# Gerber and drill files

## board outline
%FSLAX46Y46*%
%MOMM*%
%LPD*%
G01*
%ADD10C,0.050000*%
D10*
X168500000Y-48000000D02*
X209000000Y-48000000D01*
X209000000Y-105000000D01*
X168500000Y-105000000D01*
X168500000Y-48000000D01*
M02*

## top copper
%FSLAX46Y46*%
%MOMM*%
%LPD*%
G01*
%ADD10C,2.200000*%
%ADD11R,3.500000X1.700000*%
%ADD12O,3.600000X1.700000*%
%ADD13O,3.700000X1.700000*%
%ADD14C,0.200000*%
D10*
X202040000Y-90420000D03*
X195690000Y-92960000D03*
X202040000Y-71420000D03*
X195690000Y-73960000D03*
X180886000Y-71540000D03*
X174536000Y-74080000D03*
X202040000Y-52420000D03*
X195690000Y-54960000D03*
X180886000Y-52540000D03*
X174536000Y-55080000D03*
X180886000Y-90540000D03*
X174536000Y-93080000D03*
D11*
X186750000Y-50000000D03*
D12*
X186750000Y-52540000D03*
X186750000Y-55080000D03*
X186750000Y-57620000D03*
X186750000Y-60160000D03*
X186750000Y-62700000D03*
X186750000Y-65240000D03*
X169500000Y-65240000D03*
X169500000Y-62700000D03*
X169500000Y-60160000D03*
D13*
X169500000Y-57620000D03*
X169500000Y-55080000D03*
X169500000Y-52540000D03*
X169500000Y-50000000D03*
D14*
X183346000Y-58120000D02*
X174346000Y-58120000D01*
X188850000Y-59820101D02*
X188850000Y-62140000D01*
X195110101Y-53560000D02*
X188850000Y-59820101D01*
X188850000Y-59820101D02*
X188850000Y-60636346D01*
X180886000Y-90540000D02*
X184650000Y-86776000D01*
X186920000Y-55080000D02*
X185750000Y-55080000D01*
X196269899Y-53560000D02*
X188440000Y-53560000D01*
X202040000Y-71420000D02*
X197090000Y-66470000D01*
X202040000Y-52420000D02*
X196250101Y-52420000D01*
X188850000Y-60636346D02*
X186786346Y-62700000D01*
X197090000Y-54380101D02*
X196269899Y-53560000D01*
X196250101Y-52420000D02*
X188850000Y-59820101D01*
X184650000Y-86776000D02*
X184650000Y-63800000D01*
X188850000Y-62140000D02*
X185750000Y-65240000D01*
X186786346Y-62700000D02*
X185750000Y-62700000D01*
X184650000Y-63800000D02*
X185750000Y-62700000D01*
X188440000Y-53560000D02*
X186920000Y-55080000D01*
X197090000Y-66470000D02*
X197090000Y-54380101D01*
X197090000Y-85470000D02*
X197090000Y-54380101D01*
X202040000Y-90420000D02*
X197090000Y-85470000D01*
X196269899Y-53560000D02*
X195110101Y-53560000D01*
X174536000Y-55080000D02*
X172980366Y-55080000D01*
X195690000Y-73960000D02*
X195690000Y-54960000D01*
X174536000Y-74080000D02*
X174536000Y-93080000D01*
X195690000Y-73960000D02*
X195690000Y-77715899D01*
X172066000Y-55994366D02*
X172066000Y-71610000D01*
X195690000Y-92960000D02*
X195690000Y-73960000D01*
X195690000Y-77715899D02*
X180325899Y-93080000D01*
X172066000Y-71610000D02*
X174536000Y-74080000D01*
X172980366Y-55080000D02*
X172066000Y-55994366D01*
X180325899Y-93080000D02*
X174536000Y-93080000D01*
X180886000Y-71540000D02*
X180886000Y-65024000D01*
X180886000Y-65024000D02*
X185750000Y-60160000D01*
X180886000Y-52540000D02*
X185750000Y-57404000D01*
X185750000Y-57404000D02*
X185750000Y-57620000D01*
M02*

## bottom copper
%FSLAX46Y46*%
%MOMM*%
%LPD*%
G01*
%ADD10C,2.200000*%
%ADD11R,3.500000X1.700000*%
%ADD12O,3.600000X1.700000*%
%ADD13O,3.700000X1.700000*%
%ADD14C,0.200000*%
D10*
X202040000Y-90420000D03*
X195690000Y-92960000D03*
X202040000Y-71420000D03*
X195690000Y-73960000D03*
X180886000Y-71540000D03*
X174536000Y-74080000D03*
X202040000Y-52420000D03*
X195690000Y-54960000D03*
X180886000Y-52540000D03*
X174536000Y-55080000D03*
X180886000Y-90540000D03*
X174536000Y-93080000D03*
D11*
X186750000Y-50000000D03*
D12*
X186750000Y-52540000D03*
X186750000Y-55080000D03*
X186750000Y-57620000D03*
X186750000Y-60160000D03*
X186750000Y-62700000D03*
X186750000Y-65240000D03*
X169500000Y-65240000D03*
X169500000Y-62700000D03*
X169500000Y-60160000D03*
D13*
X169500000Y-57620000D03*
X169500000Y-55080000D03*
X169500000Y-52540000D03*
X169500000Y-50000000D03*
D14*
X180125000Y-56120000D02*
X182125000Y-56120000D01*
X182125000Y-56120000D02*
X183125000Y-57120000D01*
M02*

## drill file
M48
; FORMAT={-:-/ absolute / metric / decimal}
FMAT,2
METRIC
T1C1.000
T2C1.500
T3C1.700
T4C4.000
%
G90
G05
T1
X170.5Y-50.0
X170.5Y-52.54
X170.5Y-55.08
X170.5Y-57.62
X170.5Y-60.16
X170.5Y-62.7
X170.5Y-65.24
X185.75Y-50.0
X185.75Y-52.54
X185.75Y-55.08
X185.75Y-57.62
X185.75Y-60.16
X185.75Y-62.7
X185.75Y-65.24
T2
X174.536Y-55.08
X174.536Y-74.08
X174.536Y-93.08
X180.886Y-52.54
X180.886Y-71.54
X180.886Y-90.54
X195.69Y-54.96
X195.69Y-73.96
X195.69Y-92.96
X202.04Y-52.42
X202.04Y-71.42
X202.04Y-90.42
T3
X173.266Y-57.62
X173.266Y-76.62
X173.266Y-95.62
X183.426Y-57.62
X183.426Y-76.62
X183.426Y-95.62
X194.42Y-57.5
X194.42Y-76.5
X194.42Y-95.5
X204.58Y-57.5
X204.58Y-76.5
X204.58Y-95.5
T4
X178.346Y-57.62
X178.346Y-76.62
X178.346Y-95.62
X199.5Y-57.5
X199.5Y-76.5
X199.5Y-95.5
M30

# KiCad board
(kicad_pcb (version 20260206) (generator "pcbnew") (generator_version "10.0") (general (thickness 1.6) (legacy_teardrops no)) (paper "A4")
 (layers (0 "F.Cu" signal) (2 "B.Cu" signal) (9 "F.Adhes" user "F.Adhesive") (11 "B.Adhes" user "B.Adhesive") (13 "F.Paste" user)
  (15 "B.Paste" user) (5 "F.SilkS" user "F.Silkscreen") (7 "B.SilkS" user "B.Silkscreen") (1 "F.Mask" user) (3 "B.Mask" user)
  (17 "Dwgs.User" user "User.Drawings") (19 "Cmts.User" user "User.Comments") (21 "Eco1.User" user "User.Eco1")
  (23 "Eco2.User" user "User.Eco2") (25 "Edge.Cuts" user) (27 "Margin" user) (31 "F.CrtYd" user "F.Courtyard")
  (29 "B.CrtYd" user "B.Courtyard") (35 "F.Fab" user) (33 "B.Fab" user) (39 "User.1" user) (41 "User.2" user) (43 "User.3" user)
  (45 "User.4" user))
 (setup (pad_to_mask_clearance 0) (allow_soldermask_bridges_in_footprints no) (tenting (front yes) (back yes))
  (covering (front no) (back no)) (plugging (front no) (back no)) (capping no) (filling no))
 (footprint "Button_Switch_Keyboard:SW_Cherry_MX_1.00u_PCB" (layer "F.Cu") (at 202.04 90.42)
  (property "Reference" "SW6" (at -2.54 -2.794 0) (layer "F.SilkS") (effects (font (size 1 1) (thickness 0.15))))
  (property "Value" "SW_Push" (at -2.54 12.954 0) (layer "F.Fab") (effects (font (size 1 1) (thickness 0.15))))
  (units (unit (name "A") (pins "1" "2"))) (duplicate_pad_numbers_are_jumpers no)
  (pad "" np_thru_hole circle (at -7.62 5.08) (size 1.7 1.7) (drill 1.7) (layers "*.Cu" "*.Mask"))
  (pad "" np_thru_hole circle (at -2.54 5.08) (size 4 4) (drill 4) (layers "*.Cu" "*.Mask"))
  (pad "" np_thru_hole circle (at 2.54 5.08) (size 1.7 1.7) (drill 1.7) (layers "*.Cu" "*.Mask"))
  (pad "1" thru_hole circle (at 0 0) (size 2.2 2.2) (drill 1.5) (layers "*.Cu" "*.Mask") (remove_unused_layers no)
   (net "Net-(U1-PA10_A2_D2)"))
  (pad "2" thru_hole circle (at -6.35 2.54) (size 2.2 2.2) (drill 1.5) (layers "*.Cu" "*.Mask") (remove_unused_layers no) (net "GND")))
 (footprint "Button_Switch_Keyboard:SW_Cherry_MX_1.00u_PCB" (layer "F.Cu") (at 202.04 71.42)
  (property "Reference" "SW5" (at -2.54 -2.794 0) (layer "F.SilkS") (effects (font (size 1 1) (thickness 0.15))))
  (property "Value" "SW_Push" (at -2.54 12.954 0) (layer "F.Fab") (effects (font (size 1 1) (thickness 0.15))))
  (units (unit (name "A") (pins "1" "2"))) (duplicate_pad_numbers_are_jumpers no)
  (pad "" np_thru_hole circle (at -7.62 5.08) (size 1.7 1.7) (drill 1.7) (layers "*.Cu" "*.Mask"))
  (pad "" np_thru_hole circle (at -2.54 5.08) (size 4 4) (drill 4) (layers "*.Cu" "*.Mask"))
  (pad "" np_thru_hole circle (at 2.54 5.08) (size 1.7 1.7) (drill 1.7) (layers "*.Cu" "*.Mask"))
  (pad "1" thru_hole circle (at 0 0) (size 2.2 2.2) (drill 1.5) (layers "*.Cu" "*.Mask") (remove_unused_layers no)
   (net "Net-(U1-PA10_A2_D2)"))
  (pad "2" thru_hole circle (at -6.35 2.54) (size 2.2 2.2) (drill 1.5) (layers "*.Cu" "*.Mask") (remove_unused_layers no) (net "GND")))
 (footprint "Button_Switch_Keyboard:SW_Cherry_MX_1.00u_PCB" (layer "F.Cu") (at 180.886 71.54)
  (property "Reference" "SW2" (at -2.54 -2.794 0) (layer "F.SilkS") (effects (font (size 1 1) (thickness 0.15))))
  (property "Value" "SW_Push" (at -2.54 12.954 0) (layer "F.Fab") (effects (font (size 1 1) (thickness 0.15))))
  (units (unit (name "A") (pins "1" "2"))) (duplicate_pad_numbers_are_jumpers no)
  (pad "" np_thru_hole circle (at -7.62 5.08) (size 1.7 1.7) (drill 1.7) (layers "*.Cu" "*.Mask"))
  (pad "" np_thru_hole circle (at -2.54 5.08) (size 4 4) (drill 4) (layers "*.Cu" "*.Mask"))
  (pad "" np_thru_hole circle (at 2.54 5.08) (size 1.7 1.7) (drill 1.7) (layers "*.Cu" "*.Mask"))
  (pad "1" thru_hole circle (at 0 0) (size 2.2 2.2) (drill 1.5) (layers "*.Cu" "*.Mask") (remove_unused_layers no)
   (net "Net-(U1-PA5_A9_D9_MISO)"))
  (pad "2" thru_hole circle (at -6.35 2.54) (size 2.2 2.2) (drill 1.5) (layers "*.Cu" "*.Mask") (remove_unused_layers no) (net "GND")))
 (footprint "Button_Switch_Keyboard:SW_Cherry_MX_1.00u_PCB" (layer "F.Cu") (at 202.04 52.42)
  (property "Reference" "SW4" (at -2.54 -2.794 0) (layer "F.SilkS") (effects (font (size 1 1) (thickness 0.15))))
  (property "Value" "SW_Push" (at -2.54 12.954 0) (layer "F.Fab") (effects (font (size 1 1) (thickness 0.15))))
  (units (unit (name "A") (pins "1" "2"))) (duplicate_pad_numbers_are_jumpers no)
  (pad "" np_thru_hole circle (at -7.62 5.08) (size 1.7 1.7) (drill 1.7) (layers "*.Cu" "*.Mask"))
  (pad "" np_thru_hole circle (at -2.54 5.08) (size 4 4) (drill 4) (layers "*.Cu" "*.Mask"))
  (pad "" np_thru_hole circle (at 2.54 5.08) (size 1.7 1.7) (drill 1.7) (layers "*.Cu" "*.Mask"))
  (pad "1" thru_hole circle (at 0 0) (size 2.2 2.2) (drill 1.5) (layers "*.Cu" "*.Mask") (remove_unused_layers no)
   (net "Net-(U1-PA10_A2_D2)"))
  (pad "2" thru_hole circle (at -6.35 2.54) (size 2.2 2.2) (drill 1.5) (layers "*.Cu" "*.Mask") (remove_unused_layers no) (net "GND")))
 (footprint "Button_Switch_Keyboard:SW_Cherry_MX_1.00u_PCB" (layer "F.Cu") (at 180.886 52.54)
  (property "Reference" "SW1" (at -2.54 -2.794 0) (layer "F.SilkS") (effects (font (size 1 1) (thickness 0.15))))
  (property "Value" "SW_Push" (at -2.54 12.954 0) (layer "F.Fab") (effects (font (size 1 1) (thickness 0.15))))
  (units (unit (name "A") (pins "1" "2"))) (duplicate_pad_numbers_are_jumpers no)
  (pad "" np_thru_hole circle (at -7.62 5.08) (size 1.7 1.7) (drill 1.7) (layers "*.Cu" "*.Mask"))
  (pad "" np_thru_hole circle (at -2.54 5.08) (size 4 4) (drill 4) (layers "*.Cu" "*.Mask"))
  (pad "" np_thru_hole circle (at 2.54 5.08) (size 1.7 1.7) (drill 1.7) (layers "*.Cu" "*.Mask"))
  (pad "1" thru_hole circle (at 0 0) (size 2.2 2.2) (drill 1.5) (layers "*.Cu" "*.Mask") (remove_unused_layers no)
   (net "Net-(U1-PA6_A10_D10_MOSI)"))
  (pad "2" thru_hole circle (at -6.35 2.54) (size 2.2 2.2) (drill 1.5) (layers "*.Cu" "*.Mask") (remove_unused_layers no) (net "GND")))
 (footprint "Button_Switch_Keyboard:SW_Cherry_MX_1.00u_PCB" (layer "F.Cu") (at 180.886 90.54)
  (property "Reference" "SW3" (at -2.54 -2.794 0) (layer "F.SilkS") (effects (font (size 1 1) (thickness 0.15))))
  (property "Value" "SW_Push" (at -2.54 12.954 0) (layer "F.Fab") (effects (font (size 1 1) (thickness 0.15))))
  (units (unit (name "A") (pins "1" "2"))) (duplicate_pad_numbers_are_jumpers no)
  (pad "" np_thru_hole circle (at -7.62 5.08) (size 1.7 1.7) (drill 1.7) (layers "*.Cu" "*.Mask"))
  (pad "" np_thru_hole circle (at -2.54 5.08) (size 4 4) (drill 4) (layers "*.Cu" "*.Mask"))
  (pad "" np_thru_hole circle (at 2.54 5.08) (size 1.7 1.7) (drill 1.7) (layers "*.Cu" "*.Mask"))
  (pad "1" thru_hole circle (at 0 0) (size 2.2 2.2) (drill 1.5) (layers "*.Cu" "*.Mask") (remove_unused_layers no)
   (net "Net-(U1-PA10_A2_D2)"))
  (pad "2" thru_hole circle (at -6.35 2.54) (size 2.2 2.2) (drill 1.5) (layers "*.Cu" "*.Mask") (remove_unused_layers no) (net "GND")))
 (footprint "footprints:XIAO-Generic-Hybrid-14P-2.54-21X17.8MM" (layer "B.Cu") (at 178.125 57.62 180)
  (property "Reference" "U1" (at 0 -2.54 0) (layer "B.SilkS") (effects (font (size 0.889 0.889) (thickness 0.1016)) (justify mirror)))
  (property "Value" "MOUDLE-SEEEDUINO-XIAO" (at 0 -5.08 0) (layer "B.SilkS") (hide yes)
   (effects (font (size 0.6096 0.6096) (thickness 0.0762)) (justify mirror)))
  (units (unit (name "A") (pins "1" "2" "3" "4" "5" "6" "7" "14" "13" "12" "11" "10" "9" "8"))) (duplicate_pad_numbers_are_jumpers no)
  (pad "1" thru_hole rect (at -7.625 7.62 180) (size 3.5 1.7) (drill 1 (offset -1 0)) (layers "*.Cu" "*.Mask") (remove_unused_layers no)
   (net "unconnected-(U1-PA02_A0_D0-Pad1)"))
  (pad "2" thru_hole oval (at -7.625 5.08 180) (size 3.6 1.7) (drill 1 (offset -1 0)) (layers "*.Cu" "*.Mask") (remove_unused_layers no)
   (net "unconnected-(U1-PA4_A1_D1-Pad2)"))
  (pad "3" thru_hole oval (at -7.625 2.54 180) (size 3.6 1.7) (drill 1 (offset -1 0)) (layers "*.Cu" "*.Mask") (remove_unused_layers no)
   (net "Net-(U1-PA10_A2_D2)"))
  (pad "4" thru_hole oval (at -7.625 0 180) (size 3.6 1.7) (drill 1 (offset -1 0)) (layers "*.Cu" "*.Mask") (remove_unused_layers no)
   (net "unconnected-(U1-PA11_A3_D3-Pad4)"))
  (pad "5" thru_hole oval (at -7.625 -2.54 180) (size 3.6 1.7) (drill 1 (offset -1 0)) (layers "*.Cu" "*.Mask") (remove_unused_layers no)
   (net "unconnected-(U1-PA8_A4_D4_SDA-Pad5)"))
  (pad "6" thru_hole oval (at -7.625 -5.08) (size 3.6 1.7) (drill 1 (offset 1 0)) (layers "*.Cu" "*.Mask") (remove_unused_layers no)
   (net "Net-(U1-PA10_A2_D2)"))
  (pad "7" thru_hole oval (at -7.625 -7.62 180) (size 3.6 1.7) (drill 1 (offset -1 0)) (layers "*.Cu" "*.Mask") (remove_unused_layers no)
   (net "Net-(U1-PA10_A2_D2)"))
  (pad "8" thru_hole oval (at 7.625 -7.62 180) (size 3.6 1.7) (drill 1 (offset 1 0)) (layers "*.Cu" "*.Mask") (remove_unused_layers no)
   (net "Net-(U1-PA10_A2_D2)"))
  (pad "9" thru_hole oval (at 7.625 -5.08 180) (size 3.6 1.7) (drill 1 (offset 1 0)) (layers "*.Cu" "*.Mask") (remove_unused_layers no)
   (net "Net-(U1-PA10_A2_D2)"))
  (pad "10" thru_hole oval (at 7.625 -2.54 180) (size 3.6 1.7) (drill 1 (offset 1 0)) (layers "*.Cu" "*.Mask") (remove_unused_layers no)
   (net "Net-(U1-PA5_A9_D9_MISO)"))
  (pad "11" thru_hole oval (at 7.625 0 180) (size 3.7 1.7) (drill 1 (offset 1 0)) (layers "*.Cu" "*.Mask") (remove_unused_layers no)
   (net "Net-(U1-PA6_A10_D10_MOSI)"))
  (pad "12" thru_hole oval (at 7.625 2.54 180) (size 3.7 1.7) (drill 1 (offset 1 0)) (layers "*.Cu" "*.Mask") (remove_unused_layers no)
   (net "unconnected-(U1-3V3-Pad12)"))
  (pad "13" thru_hole oval (at 7.625 5.08 180) (size 3.7 1.7) (drill 1 (offset 1 0)) (layers "*.Cu" "*.Mask") (remove_unused_layers no)
   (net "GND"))
  (pad "14" thru_hole oval (at 7.625 7.62 180) (size 3.7 1.7) (drill 1 (offset 1 0)) (layers "*.Cu" "*.Mask") (remove_unused_layers no)
   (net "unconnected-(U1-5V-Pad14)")))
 (gr_rect (start 168.5 48) (end 209 105) (stroke (width 0.05) (type default)) (fill no) (layer "Edge.Cuts"))
 (segment (start 183.346 58.12) (end 174.346 58.12) (width 0.2) (layer "F.Cu") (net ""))
 (segment (start 180.125 56.12) (end 182.125 56.12) (width 0.2) (layer "B.Cu") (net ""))
 (segment (start 182.125 56.12) (end 183.125 57.12) (width 0.2) (layer "B.Cu") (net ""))
 (segment (start 188.85 59.820101) (end 188.85 62.14) (width 0.2) (layer "F.Cu") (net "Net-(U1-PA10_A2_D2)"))
 (segment (start 195.110101 53.56) (end 188.85 59.820101) (width 0.2) (layer "F.Cu") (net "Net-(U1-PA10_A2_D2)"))
 (segment (start 188.85 59.820101) (end 188.85 60.636346) (width 0.2) (layer "F.Cu") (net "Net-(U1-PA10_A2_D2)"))
 (segment (start 180.886 90.54) (end 184.65 86.776) (width 0.2) (layer "F.Cu") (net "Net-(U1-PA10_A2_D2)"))
 (segment (start 186.92 55.08) (end 185.75 55.08) (width 0.2) (layer "F.Cu") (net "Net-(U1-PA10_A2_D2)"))
 (segment (start 196.269899 53.56) (end 188.44 53.56) (width 0.2) (layer "F.Cu") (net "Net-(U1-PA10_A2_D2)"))
 (segment (start 202.04 71.42) (end 197.09 66.47) (width 0.2) (layer "F.Cu") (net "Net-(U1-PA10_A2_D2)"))
 (segment (start 202.04 52.42) (end 196.250101 52.42) (width 0.2) (layer "F.Cu") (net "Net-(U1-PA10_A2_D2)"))
 (segment (start 188.85 60.636346) (end 186.786346 62.7) (width 0.2) (layer "F.Cu") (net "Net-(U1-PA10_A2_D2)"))
 (segment (start 197.09 54.380101) (end 196.269899 53.56) (width 0.2) (layer "F.Cu") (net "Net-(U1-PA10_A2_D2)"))
 (segment (start 196.250101 52.42) (end 188.85 59.820101) (width 0.2) (layer "F.Cu") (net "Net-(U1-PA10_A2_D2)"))
 (segment (start 184.65 86.776) (end 184.65 63.8) (width 0.2) (layer "F.Cu") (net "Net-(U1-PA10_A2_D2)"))
 (segment (start 188.85 62.14) (end 185.75 65.24) (width 0.2) (layer "F.Cu") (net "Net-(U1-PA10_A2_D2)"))
 (segment (start 186.786346 62.7) (end 185.75 62.7) (width 0.2) (layer "F.Cu") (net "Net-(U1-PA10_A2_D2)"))
 (segment (start 184.65 63.8) (end 185.75 62.7) (width 0.2) (layer "F.Cu") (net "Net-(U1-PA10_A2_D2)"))
 (segment (start 188.44 53.56) (end 186.92 55.08) (width 0.2) (layer "F.Cu") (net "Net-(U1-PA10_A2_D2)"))
 (segment (start 197.09 66.47) (end 197.09 54.380101) (width 0.2) (layer "F.Cu") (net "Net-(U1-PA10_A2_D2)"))
 (segment (start 197.09 85.47) (end 197.09 54.380101) (width 0.2) (layer "F.Cu") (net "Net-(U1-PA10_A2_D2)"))
 (segment (start 202.04 90.42) (end 197.09 85.47) (width 0.2) (layer "F.Cu") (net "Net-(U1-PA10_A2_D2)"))
 (segment (start 196.269899 53.56) (end 195.110101 53.56) (width 0.2) (layer "F.Cu") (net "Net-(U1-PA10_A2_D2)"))
 (segment (start 174.536 55.08) (end 172.980366 55.08) (width 0.2) (layer "F.Cu") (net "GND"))
 (segment (start 195.69 73.96) (end 195.69 54.96) (width 0.2) (layer "F.Cu") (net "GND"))
 (segment (start 174.536 74.08) (end 174.536 93.08) (width 0.2) (layer "F.Cu") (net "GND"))
 (segment (start 195.69 73.96) (end 195.69 77.715899) (width 0.2) (layer "F.Cu") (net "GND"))
 (segment (start 172.066 55.994366) (end 172.066 71.61) (width 0.2) (layer "F.Cu") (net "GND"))
 (segment (start 195.69 92.96) (end 195.69 73.96) (width 0.2) (layer "F.Cu") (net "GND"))
 (segment (start 195.69 77.715899) (end 180.325899 93.08) (width 0.2) (layer "F.Cu") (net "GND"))
 (segment (start 172.066 71.61) (end 174.536 74.08) (width 0.2) (layer "F.Cu") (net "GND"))
 (segment (start 172.980366 55.08) (end 172.066 55.994366) (width 0.2) (layer "F.Cu") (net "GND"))
 (segment (start 180.325899 93.08) (end 174.536 93.08) (width 0.2) (layer "F.Cu") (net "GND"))
 (segment (start 180.886 71.54) (end 180.886 65.024) (width 0.2) (layer "F.Cu") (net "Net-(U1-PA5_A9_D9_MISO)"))
 (segment (start 180.886 65.024) (end 185.75 60.16) (width 0.2) (layer "F.Cu") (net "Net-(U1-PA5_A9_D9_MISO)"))
 (segment (start 180.886 52.54) (end 185.75 57.404) (width 0.2) (layer "F.Cu") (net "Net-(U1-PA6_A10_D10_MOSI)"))
 (segment (start 185.75 57.404) (end 185.75 57.62) (width 0.2) (layer "F.Cu") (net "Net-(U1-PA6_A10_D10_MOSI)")))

